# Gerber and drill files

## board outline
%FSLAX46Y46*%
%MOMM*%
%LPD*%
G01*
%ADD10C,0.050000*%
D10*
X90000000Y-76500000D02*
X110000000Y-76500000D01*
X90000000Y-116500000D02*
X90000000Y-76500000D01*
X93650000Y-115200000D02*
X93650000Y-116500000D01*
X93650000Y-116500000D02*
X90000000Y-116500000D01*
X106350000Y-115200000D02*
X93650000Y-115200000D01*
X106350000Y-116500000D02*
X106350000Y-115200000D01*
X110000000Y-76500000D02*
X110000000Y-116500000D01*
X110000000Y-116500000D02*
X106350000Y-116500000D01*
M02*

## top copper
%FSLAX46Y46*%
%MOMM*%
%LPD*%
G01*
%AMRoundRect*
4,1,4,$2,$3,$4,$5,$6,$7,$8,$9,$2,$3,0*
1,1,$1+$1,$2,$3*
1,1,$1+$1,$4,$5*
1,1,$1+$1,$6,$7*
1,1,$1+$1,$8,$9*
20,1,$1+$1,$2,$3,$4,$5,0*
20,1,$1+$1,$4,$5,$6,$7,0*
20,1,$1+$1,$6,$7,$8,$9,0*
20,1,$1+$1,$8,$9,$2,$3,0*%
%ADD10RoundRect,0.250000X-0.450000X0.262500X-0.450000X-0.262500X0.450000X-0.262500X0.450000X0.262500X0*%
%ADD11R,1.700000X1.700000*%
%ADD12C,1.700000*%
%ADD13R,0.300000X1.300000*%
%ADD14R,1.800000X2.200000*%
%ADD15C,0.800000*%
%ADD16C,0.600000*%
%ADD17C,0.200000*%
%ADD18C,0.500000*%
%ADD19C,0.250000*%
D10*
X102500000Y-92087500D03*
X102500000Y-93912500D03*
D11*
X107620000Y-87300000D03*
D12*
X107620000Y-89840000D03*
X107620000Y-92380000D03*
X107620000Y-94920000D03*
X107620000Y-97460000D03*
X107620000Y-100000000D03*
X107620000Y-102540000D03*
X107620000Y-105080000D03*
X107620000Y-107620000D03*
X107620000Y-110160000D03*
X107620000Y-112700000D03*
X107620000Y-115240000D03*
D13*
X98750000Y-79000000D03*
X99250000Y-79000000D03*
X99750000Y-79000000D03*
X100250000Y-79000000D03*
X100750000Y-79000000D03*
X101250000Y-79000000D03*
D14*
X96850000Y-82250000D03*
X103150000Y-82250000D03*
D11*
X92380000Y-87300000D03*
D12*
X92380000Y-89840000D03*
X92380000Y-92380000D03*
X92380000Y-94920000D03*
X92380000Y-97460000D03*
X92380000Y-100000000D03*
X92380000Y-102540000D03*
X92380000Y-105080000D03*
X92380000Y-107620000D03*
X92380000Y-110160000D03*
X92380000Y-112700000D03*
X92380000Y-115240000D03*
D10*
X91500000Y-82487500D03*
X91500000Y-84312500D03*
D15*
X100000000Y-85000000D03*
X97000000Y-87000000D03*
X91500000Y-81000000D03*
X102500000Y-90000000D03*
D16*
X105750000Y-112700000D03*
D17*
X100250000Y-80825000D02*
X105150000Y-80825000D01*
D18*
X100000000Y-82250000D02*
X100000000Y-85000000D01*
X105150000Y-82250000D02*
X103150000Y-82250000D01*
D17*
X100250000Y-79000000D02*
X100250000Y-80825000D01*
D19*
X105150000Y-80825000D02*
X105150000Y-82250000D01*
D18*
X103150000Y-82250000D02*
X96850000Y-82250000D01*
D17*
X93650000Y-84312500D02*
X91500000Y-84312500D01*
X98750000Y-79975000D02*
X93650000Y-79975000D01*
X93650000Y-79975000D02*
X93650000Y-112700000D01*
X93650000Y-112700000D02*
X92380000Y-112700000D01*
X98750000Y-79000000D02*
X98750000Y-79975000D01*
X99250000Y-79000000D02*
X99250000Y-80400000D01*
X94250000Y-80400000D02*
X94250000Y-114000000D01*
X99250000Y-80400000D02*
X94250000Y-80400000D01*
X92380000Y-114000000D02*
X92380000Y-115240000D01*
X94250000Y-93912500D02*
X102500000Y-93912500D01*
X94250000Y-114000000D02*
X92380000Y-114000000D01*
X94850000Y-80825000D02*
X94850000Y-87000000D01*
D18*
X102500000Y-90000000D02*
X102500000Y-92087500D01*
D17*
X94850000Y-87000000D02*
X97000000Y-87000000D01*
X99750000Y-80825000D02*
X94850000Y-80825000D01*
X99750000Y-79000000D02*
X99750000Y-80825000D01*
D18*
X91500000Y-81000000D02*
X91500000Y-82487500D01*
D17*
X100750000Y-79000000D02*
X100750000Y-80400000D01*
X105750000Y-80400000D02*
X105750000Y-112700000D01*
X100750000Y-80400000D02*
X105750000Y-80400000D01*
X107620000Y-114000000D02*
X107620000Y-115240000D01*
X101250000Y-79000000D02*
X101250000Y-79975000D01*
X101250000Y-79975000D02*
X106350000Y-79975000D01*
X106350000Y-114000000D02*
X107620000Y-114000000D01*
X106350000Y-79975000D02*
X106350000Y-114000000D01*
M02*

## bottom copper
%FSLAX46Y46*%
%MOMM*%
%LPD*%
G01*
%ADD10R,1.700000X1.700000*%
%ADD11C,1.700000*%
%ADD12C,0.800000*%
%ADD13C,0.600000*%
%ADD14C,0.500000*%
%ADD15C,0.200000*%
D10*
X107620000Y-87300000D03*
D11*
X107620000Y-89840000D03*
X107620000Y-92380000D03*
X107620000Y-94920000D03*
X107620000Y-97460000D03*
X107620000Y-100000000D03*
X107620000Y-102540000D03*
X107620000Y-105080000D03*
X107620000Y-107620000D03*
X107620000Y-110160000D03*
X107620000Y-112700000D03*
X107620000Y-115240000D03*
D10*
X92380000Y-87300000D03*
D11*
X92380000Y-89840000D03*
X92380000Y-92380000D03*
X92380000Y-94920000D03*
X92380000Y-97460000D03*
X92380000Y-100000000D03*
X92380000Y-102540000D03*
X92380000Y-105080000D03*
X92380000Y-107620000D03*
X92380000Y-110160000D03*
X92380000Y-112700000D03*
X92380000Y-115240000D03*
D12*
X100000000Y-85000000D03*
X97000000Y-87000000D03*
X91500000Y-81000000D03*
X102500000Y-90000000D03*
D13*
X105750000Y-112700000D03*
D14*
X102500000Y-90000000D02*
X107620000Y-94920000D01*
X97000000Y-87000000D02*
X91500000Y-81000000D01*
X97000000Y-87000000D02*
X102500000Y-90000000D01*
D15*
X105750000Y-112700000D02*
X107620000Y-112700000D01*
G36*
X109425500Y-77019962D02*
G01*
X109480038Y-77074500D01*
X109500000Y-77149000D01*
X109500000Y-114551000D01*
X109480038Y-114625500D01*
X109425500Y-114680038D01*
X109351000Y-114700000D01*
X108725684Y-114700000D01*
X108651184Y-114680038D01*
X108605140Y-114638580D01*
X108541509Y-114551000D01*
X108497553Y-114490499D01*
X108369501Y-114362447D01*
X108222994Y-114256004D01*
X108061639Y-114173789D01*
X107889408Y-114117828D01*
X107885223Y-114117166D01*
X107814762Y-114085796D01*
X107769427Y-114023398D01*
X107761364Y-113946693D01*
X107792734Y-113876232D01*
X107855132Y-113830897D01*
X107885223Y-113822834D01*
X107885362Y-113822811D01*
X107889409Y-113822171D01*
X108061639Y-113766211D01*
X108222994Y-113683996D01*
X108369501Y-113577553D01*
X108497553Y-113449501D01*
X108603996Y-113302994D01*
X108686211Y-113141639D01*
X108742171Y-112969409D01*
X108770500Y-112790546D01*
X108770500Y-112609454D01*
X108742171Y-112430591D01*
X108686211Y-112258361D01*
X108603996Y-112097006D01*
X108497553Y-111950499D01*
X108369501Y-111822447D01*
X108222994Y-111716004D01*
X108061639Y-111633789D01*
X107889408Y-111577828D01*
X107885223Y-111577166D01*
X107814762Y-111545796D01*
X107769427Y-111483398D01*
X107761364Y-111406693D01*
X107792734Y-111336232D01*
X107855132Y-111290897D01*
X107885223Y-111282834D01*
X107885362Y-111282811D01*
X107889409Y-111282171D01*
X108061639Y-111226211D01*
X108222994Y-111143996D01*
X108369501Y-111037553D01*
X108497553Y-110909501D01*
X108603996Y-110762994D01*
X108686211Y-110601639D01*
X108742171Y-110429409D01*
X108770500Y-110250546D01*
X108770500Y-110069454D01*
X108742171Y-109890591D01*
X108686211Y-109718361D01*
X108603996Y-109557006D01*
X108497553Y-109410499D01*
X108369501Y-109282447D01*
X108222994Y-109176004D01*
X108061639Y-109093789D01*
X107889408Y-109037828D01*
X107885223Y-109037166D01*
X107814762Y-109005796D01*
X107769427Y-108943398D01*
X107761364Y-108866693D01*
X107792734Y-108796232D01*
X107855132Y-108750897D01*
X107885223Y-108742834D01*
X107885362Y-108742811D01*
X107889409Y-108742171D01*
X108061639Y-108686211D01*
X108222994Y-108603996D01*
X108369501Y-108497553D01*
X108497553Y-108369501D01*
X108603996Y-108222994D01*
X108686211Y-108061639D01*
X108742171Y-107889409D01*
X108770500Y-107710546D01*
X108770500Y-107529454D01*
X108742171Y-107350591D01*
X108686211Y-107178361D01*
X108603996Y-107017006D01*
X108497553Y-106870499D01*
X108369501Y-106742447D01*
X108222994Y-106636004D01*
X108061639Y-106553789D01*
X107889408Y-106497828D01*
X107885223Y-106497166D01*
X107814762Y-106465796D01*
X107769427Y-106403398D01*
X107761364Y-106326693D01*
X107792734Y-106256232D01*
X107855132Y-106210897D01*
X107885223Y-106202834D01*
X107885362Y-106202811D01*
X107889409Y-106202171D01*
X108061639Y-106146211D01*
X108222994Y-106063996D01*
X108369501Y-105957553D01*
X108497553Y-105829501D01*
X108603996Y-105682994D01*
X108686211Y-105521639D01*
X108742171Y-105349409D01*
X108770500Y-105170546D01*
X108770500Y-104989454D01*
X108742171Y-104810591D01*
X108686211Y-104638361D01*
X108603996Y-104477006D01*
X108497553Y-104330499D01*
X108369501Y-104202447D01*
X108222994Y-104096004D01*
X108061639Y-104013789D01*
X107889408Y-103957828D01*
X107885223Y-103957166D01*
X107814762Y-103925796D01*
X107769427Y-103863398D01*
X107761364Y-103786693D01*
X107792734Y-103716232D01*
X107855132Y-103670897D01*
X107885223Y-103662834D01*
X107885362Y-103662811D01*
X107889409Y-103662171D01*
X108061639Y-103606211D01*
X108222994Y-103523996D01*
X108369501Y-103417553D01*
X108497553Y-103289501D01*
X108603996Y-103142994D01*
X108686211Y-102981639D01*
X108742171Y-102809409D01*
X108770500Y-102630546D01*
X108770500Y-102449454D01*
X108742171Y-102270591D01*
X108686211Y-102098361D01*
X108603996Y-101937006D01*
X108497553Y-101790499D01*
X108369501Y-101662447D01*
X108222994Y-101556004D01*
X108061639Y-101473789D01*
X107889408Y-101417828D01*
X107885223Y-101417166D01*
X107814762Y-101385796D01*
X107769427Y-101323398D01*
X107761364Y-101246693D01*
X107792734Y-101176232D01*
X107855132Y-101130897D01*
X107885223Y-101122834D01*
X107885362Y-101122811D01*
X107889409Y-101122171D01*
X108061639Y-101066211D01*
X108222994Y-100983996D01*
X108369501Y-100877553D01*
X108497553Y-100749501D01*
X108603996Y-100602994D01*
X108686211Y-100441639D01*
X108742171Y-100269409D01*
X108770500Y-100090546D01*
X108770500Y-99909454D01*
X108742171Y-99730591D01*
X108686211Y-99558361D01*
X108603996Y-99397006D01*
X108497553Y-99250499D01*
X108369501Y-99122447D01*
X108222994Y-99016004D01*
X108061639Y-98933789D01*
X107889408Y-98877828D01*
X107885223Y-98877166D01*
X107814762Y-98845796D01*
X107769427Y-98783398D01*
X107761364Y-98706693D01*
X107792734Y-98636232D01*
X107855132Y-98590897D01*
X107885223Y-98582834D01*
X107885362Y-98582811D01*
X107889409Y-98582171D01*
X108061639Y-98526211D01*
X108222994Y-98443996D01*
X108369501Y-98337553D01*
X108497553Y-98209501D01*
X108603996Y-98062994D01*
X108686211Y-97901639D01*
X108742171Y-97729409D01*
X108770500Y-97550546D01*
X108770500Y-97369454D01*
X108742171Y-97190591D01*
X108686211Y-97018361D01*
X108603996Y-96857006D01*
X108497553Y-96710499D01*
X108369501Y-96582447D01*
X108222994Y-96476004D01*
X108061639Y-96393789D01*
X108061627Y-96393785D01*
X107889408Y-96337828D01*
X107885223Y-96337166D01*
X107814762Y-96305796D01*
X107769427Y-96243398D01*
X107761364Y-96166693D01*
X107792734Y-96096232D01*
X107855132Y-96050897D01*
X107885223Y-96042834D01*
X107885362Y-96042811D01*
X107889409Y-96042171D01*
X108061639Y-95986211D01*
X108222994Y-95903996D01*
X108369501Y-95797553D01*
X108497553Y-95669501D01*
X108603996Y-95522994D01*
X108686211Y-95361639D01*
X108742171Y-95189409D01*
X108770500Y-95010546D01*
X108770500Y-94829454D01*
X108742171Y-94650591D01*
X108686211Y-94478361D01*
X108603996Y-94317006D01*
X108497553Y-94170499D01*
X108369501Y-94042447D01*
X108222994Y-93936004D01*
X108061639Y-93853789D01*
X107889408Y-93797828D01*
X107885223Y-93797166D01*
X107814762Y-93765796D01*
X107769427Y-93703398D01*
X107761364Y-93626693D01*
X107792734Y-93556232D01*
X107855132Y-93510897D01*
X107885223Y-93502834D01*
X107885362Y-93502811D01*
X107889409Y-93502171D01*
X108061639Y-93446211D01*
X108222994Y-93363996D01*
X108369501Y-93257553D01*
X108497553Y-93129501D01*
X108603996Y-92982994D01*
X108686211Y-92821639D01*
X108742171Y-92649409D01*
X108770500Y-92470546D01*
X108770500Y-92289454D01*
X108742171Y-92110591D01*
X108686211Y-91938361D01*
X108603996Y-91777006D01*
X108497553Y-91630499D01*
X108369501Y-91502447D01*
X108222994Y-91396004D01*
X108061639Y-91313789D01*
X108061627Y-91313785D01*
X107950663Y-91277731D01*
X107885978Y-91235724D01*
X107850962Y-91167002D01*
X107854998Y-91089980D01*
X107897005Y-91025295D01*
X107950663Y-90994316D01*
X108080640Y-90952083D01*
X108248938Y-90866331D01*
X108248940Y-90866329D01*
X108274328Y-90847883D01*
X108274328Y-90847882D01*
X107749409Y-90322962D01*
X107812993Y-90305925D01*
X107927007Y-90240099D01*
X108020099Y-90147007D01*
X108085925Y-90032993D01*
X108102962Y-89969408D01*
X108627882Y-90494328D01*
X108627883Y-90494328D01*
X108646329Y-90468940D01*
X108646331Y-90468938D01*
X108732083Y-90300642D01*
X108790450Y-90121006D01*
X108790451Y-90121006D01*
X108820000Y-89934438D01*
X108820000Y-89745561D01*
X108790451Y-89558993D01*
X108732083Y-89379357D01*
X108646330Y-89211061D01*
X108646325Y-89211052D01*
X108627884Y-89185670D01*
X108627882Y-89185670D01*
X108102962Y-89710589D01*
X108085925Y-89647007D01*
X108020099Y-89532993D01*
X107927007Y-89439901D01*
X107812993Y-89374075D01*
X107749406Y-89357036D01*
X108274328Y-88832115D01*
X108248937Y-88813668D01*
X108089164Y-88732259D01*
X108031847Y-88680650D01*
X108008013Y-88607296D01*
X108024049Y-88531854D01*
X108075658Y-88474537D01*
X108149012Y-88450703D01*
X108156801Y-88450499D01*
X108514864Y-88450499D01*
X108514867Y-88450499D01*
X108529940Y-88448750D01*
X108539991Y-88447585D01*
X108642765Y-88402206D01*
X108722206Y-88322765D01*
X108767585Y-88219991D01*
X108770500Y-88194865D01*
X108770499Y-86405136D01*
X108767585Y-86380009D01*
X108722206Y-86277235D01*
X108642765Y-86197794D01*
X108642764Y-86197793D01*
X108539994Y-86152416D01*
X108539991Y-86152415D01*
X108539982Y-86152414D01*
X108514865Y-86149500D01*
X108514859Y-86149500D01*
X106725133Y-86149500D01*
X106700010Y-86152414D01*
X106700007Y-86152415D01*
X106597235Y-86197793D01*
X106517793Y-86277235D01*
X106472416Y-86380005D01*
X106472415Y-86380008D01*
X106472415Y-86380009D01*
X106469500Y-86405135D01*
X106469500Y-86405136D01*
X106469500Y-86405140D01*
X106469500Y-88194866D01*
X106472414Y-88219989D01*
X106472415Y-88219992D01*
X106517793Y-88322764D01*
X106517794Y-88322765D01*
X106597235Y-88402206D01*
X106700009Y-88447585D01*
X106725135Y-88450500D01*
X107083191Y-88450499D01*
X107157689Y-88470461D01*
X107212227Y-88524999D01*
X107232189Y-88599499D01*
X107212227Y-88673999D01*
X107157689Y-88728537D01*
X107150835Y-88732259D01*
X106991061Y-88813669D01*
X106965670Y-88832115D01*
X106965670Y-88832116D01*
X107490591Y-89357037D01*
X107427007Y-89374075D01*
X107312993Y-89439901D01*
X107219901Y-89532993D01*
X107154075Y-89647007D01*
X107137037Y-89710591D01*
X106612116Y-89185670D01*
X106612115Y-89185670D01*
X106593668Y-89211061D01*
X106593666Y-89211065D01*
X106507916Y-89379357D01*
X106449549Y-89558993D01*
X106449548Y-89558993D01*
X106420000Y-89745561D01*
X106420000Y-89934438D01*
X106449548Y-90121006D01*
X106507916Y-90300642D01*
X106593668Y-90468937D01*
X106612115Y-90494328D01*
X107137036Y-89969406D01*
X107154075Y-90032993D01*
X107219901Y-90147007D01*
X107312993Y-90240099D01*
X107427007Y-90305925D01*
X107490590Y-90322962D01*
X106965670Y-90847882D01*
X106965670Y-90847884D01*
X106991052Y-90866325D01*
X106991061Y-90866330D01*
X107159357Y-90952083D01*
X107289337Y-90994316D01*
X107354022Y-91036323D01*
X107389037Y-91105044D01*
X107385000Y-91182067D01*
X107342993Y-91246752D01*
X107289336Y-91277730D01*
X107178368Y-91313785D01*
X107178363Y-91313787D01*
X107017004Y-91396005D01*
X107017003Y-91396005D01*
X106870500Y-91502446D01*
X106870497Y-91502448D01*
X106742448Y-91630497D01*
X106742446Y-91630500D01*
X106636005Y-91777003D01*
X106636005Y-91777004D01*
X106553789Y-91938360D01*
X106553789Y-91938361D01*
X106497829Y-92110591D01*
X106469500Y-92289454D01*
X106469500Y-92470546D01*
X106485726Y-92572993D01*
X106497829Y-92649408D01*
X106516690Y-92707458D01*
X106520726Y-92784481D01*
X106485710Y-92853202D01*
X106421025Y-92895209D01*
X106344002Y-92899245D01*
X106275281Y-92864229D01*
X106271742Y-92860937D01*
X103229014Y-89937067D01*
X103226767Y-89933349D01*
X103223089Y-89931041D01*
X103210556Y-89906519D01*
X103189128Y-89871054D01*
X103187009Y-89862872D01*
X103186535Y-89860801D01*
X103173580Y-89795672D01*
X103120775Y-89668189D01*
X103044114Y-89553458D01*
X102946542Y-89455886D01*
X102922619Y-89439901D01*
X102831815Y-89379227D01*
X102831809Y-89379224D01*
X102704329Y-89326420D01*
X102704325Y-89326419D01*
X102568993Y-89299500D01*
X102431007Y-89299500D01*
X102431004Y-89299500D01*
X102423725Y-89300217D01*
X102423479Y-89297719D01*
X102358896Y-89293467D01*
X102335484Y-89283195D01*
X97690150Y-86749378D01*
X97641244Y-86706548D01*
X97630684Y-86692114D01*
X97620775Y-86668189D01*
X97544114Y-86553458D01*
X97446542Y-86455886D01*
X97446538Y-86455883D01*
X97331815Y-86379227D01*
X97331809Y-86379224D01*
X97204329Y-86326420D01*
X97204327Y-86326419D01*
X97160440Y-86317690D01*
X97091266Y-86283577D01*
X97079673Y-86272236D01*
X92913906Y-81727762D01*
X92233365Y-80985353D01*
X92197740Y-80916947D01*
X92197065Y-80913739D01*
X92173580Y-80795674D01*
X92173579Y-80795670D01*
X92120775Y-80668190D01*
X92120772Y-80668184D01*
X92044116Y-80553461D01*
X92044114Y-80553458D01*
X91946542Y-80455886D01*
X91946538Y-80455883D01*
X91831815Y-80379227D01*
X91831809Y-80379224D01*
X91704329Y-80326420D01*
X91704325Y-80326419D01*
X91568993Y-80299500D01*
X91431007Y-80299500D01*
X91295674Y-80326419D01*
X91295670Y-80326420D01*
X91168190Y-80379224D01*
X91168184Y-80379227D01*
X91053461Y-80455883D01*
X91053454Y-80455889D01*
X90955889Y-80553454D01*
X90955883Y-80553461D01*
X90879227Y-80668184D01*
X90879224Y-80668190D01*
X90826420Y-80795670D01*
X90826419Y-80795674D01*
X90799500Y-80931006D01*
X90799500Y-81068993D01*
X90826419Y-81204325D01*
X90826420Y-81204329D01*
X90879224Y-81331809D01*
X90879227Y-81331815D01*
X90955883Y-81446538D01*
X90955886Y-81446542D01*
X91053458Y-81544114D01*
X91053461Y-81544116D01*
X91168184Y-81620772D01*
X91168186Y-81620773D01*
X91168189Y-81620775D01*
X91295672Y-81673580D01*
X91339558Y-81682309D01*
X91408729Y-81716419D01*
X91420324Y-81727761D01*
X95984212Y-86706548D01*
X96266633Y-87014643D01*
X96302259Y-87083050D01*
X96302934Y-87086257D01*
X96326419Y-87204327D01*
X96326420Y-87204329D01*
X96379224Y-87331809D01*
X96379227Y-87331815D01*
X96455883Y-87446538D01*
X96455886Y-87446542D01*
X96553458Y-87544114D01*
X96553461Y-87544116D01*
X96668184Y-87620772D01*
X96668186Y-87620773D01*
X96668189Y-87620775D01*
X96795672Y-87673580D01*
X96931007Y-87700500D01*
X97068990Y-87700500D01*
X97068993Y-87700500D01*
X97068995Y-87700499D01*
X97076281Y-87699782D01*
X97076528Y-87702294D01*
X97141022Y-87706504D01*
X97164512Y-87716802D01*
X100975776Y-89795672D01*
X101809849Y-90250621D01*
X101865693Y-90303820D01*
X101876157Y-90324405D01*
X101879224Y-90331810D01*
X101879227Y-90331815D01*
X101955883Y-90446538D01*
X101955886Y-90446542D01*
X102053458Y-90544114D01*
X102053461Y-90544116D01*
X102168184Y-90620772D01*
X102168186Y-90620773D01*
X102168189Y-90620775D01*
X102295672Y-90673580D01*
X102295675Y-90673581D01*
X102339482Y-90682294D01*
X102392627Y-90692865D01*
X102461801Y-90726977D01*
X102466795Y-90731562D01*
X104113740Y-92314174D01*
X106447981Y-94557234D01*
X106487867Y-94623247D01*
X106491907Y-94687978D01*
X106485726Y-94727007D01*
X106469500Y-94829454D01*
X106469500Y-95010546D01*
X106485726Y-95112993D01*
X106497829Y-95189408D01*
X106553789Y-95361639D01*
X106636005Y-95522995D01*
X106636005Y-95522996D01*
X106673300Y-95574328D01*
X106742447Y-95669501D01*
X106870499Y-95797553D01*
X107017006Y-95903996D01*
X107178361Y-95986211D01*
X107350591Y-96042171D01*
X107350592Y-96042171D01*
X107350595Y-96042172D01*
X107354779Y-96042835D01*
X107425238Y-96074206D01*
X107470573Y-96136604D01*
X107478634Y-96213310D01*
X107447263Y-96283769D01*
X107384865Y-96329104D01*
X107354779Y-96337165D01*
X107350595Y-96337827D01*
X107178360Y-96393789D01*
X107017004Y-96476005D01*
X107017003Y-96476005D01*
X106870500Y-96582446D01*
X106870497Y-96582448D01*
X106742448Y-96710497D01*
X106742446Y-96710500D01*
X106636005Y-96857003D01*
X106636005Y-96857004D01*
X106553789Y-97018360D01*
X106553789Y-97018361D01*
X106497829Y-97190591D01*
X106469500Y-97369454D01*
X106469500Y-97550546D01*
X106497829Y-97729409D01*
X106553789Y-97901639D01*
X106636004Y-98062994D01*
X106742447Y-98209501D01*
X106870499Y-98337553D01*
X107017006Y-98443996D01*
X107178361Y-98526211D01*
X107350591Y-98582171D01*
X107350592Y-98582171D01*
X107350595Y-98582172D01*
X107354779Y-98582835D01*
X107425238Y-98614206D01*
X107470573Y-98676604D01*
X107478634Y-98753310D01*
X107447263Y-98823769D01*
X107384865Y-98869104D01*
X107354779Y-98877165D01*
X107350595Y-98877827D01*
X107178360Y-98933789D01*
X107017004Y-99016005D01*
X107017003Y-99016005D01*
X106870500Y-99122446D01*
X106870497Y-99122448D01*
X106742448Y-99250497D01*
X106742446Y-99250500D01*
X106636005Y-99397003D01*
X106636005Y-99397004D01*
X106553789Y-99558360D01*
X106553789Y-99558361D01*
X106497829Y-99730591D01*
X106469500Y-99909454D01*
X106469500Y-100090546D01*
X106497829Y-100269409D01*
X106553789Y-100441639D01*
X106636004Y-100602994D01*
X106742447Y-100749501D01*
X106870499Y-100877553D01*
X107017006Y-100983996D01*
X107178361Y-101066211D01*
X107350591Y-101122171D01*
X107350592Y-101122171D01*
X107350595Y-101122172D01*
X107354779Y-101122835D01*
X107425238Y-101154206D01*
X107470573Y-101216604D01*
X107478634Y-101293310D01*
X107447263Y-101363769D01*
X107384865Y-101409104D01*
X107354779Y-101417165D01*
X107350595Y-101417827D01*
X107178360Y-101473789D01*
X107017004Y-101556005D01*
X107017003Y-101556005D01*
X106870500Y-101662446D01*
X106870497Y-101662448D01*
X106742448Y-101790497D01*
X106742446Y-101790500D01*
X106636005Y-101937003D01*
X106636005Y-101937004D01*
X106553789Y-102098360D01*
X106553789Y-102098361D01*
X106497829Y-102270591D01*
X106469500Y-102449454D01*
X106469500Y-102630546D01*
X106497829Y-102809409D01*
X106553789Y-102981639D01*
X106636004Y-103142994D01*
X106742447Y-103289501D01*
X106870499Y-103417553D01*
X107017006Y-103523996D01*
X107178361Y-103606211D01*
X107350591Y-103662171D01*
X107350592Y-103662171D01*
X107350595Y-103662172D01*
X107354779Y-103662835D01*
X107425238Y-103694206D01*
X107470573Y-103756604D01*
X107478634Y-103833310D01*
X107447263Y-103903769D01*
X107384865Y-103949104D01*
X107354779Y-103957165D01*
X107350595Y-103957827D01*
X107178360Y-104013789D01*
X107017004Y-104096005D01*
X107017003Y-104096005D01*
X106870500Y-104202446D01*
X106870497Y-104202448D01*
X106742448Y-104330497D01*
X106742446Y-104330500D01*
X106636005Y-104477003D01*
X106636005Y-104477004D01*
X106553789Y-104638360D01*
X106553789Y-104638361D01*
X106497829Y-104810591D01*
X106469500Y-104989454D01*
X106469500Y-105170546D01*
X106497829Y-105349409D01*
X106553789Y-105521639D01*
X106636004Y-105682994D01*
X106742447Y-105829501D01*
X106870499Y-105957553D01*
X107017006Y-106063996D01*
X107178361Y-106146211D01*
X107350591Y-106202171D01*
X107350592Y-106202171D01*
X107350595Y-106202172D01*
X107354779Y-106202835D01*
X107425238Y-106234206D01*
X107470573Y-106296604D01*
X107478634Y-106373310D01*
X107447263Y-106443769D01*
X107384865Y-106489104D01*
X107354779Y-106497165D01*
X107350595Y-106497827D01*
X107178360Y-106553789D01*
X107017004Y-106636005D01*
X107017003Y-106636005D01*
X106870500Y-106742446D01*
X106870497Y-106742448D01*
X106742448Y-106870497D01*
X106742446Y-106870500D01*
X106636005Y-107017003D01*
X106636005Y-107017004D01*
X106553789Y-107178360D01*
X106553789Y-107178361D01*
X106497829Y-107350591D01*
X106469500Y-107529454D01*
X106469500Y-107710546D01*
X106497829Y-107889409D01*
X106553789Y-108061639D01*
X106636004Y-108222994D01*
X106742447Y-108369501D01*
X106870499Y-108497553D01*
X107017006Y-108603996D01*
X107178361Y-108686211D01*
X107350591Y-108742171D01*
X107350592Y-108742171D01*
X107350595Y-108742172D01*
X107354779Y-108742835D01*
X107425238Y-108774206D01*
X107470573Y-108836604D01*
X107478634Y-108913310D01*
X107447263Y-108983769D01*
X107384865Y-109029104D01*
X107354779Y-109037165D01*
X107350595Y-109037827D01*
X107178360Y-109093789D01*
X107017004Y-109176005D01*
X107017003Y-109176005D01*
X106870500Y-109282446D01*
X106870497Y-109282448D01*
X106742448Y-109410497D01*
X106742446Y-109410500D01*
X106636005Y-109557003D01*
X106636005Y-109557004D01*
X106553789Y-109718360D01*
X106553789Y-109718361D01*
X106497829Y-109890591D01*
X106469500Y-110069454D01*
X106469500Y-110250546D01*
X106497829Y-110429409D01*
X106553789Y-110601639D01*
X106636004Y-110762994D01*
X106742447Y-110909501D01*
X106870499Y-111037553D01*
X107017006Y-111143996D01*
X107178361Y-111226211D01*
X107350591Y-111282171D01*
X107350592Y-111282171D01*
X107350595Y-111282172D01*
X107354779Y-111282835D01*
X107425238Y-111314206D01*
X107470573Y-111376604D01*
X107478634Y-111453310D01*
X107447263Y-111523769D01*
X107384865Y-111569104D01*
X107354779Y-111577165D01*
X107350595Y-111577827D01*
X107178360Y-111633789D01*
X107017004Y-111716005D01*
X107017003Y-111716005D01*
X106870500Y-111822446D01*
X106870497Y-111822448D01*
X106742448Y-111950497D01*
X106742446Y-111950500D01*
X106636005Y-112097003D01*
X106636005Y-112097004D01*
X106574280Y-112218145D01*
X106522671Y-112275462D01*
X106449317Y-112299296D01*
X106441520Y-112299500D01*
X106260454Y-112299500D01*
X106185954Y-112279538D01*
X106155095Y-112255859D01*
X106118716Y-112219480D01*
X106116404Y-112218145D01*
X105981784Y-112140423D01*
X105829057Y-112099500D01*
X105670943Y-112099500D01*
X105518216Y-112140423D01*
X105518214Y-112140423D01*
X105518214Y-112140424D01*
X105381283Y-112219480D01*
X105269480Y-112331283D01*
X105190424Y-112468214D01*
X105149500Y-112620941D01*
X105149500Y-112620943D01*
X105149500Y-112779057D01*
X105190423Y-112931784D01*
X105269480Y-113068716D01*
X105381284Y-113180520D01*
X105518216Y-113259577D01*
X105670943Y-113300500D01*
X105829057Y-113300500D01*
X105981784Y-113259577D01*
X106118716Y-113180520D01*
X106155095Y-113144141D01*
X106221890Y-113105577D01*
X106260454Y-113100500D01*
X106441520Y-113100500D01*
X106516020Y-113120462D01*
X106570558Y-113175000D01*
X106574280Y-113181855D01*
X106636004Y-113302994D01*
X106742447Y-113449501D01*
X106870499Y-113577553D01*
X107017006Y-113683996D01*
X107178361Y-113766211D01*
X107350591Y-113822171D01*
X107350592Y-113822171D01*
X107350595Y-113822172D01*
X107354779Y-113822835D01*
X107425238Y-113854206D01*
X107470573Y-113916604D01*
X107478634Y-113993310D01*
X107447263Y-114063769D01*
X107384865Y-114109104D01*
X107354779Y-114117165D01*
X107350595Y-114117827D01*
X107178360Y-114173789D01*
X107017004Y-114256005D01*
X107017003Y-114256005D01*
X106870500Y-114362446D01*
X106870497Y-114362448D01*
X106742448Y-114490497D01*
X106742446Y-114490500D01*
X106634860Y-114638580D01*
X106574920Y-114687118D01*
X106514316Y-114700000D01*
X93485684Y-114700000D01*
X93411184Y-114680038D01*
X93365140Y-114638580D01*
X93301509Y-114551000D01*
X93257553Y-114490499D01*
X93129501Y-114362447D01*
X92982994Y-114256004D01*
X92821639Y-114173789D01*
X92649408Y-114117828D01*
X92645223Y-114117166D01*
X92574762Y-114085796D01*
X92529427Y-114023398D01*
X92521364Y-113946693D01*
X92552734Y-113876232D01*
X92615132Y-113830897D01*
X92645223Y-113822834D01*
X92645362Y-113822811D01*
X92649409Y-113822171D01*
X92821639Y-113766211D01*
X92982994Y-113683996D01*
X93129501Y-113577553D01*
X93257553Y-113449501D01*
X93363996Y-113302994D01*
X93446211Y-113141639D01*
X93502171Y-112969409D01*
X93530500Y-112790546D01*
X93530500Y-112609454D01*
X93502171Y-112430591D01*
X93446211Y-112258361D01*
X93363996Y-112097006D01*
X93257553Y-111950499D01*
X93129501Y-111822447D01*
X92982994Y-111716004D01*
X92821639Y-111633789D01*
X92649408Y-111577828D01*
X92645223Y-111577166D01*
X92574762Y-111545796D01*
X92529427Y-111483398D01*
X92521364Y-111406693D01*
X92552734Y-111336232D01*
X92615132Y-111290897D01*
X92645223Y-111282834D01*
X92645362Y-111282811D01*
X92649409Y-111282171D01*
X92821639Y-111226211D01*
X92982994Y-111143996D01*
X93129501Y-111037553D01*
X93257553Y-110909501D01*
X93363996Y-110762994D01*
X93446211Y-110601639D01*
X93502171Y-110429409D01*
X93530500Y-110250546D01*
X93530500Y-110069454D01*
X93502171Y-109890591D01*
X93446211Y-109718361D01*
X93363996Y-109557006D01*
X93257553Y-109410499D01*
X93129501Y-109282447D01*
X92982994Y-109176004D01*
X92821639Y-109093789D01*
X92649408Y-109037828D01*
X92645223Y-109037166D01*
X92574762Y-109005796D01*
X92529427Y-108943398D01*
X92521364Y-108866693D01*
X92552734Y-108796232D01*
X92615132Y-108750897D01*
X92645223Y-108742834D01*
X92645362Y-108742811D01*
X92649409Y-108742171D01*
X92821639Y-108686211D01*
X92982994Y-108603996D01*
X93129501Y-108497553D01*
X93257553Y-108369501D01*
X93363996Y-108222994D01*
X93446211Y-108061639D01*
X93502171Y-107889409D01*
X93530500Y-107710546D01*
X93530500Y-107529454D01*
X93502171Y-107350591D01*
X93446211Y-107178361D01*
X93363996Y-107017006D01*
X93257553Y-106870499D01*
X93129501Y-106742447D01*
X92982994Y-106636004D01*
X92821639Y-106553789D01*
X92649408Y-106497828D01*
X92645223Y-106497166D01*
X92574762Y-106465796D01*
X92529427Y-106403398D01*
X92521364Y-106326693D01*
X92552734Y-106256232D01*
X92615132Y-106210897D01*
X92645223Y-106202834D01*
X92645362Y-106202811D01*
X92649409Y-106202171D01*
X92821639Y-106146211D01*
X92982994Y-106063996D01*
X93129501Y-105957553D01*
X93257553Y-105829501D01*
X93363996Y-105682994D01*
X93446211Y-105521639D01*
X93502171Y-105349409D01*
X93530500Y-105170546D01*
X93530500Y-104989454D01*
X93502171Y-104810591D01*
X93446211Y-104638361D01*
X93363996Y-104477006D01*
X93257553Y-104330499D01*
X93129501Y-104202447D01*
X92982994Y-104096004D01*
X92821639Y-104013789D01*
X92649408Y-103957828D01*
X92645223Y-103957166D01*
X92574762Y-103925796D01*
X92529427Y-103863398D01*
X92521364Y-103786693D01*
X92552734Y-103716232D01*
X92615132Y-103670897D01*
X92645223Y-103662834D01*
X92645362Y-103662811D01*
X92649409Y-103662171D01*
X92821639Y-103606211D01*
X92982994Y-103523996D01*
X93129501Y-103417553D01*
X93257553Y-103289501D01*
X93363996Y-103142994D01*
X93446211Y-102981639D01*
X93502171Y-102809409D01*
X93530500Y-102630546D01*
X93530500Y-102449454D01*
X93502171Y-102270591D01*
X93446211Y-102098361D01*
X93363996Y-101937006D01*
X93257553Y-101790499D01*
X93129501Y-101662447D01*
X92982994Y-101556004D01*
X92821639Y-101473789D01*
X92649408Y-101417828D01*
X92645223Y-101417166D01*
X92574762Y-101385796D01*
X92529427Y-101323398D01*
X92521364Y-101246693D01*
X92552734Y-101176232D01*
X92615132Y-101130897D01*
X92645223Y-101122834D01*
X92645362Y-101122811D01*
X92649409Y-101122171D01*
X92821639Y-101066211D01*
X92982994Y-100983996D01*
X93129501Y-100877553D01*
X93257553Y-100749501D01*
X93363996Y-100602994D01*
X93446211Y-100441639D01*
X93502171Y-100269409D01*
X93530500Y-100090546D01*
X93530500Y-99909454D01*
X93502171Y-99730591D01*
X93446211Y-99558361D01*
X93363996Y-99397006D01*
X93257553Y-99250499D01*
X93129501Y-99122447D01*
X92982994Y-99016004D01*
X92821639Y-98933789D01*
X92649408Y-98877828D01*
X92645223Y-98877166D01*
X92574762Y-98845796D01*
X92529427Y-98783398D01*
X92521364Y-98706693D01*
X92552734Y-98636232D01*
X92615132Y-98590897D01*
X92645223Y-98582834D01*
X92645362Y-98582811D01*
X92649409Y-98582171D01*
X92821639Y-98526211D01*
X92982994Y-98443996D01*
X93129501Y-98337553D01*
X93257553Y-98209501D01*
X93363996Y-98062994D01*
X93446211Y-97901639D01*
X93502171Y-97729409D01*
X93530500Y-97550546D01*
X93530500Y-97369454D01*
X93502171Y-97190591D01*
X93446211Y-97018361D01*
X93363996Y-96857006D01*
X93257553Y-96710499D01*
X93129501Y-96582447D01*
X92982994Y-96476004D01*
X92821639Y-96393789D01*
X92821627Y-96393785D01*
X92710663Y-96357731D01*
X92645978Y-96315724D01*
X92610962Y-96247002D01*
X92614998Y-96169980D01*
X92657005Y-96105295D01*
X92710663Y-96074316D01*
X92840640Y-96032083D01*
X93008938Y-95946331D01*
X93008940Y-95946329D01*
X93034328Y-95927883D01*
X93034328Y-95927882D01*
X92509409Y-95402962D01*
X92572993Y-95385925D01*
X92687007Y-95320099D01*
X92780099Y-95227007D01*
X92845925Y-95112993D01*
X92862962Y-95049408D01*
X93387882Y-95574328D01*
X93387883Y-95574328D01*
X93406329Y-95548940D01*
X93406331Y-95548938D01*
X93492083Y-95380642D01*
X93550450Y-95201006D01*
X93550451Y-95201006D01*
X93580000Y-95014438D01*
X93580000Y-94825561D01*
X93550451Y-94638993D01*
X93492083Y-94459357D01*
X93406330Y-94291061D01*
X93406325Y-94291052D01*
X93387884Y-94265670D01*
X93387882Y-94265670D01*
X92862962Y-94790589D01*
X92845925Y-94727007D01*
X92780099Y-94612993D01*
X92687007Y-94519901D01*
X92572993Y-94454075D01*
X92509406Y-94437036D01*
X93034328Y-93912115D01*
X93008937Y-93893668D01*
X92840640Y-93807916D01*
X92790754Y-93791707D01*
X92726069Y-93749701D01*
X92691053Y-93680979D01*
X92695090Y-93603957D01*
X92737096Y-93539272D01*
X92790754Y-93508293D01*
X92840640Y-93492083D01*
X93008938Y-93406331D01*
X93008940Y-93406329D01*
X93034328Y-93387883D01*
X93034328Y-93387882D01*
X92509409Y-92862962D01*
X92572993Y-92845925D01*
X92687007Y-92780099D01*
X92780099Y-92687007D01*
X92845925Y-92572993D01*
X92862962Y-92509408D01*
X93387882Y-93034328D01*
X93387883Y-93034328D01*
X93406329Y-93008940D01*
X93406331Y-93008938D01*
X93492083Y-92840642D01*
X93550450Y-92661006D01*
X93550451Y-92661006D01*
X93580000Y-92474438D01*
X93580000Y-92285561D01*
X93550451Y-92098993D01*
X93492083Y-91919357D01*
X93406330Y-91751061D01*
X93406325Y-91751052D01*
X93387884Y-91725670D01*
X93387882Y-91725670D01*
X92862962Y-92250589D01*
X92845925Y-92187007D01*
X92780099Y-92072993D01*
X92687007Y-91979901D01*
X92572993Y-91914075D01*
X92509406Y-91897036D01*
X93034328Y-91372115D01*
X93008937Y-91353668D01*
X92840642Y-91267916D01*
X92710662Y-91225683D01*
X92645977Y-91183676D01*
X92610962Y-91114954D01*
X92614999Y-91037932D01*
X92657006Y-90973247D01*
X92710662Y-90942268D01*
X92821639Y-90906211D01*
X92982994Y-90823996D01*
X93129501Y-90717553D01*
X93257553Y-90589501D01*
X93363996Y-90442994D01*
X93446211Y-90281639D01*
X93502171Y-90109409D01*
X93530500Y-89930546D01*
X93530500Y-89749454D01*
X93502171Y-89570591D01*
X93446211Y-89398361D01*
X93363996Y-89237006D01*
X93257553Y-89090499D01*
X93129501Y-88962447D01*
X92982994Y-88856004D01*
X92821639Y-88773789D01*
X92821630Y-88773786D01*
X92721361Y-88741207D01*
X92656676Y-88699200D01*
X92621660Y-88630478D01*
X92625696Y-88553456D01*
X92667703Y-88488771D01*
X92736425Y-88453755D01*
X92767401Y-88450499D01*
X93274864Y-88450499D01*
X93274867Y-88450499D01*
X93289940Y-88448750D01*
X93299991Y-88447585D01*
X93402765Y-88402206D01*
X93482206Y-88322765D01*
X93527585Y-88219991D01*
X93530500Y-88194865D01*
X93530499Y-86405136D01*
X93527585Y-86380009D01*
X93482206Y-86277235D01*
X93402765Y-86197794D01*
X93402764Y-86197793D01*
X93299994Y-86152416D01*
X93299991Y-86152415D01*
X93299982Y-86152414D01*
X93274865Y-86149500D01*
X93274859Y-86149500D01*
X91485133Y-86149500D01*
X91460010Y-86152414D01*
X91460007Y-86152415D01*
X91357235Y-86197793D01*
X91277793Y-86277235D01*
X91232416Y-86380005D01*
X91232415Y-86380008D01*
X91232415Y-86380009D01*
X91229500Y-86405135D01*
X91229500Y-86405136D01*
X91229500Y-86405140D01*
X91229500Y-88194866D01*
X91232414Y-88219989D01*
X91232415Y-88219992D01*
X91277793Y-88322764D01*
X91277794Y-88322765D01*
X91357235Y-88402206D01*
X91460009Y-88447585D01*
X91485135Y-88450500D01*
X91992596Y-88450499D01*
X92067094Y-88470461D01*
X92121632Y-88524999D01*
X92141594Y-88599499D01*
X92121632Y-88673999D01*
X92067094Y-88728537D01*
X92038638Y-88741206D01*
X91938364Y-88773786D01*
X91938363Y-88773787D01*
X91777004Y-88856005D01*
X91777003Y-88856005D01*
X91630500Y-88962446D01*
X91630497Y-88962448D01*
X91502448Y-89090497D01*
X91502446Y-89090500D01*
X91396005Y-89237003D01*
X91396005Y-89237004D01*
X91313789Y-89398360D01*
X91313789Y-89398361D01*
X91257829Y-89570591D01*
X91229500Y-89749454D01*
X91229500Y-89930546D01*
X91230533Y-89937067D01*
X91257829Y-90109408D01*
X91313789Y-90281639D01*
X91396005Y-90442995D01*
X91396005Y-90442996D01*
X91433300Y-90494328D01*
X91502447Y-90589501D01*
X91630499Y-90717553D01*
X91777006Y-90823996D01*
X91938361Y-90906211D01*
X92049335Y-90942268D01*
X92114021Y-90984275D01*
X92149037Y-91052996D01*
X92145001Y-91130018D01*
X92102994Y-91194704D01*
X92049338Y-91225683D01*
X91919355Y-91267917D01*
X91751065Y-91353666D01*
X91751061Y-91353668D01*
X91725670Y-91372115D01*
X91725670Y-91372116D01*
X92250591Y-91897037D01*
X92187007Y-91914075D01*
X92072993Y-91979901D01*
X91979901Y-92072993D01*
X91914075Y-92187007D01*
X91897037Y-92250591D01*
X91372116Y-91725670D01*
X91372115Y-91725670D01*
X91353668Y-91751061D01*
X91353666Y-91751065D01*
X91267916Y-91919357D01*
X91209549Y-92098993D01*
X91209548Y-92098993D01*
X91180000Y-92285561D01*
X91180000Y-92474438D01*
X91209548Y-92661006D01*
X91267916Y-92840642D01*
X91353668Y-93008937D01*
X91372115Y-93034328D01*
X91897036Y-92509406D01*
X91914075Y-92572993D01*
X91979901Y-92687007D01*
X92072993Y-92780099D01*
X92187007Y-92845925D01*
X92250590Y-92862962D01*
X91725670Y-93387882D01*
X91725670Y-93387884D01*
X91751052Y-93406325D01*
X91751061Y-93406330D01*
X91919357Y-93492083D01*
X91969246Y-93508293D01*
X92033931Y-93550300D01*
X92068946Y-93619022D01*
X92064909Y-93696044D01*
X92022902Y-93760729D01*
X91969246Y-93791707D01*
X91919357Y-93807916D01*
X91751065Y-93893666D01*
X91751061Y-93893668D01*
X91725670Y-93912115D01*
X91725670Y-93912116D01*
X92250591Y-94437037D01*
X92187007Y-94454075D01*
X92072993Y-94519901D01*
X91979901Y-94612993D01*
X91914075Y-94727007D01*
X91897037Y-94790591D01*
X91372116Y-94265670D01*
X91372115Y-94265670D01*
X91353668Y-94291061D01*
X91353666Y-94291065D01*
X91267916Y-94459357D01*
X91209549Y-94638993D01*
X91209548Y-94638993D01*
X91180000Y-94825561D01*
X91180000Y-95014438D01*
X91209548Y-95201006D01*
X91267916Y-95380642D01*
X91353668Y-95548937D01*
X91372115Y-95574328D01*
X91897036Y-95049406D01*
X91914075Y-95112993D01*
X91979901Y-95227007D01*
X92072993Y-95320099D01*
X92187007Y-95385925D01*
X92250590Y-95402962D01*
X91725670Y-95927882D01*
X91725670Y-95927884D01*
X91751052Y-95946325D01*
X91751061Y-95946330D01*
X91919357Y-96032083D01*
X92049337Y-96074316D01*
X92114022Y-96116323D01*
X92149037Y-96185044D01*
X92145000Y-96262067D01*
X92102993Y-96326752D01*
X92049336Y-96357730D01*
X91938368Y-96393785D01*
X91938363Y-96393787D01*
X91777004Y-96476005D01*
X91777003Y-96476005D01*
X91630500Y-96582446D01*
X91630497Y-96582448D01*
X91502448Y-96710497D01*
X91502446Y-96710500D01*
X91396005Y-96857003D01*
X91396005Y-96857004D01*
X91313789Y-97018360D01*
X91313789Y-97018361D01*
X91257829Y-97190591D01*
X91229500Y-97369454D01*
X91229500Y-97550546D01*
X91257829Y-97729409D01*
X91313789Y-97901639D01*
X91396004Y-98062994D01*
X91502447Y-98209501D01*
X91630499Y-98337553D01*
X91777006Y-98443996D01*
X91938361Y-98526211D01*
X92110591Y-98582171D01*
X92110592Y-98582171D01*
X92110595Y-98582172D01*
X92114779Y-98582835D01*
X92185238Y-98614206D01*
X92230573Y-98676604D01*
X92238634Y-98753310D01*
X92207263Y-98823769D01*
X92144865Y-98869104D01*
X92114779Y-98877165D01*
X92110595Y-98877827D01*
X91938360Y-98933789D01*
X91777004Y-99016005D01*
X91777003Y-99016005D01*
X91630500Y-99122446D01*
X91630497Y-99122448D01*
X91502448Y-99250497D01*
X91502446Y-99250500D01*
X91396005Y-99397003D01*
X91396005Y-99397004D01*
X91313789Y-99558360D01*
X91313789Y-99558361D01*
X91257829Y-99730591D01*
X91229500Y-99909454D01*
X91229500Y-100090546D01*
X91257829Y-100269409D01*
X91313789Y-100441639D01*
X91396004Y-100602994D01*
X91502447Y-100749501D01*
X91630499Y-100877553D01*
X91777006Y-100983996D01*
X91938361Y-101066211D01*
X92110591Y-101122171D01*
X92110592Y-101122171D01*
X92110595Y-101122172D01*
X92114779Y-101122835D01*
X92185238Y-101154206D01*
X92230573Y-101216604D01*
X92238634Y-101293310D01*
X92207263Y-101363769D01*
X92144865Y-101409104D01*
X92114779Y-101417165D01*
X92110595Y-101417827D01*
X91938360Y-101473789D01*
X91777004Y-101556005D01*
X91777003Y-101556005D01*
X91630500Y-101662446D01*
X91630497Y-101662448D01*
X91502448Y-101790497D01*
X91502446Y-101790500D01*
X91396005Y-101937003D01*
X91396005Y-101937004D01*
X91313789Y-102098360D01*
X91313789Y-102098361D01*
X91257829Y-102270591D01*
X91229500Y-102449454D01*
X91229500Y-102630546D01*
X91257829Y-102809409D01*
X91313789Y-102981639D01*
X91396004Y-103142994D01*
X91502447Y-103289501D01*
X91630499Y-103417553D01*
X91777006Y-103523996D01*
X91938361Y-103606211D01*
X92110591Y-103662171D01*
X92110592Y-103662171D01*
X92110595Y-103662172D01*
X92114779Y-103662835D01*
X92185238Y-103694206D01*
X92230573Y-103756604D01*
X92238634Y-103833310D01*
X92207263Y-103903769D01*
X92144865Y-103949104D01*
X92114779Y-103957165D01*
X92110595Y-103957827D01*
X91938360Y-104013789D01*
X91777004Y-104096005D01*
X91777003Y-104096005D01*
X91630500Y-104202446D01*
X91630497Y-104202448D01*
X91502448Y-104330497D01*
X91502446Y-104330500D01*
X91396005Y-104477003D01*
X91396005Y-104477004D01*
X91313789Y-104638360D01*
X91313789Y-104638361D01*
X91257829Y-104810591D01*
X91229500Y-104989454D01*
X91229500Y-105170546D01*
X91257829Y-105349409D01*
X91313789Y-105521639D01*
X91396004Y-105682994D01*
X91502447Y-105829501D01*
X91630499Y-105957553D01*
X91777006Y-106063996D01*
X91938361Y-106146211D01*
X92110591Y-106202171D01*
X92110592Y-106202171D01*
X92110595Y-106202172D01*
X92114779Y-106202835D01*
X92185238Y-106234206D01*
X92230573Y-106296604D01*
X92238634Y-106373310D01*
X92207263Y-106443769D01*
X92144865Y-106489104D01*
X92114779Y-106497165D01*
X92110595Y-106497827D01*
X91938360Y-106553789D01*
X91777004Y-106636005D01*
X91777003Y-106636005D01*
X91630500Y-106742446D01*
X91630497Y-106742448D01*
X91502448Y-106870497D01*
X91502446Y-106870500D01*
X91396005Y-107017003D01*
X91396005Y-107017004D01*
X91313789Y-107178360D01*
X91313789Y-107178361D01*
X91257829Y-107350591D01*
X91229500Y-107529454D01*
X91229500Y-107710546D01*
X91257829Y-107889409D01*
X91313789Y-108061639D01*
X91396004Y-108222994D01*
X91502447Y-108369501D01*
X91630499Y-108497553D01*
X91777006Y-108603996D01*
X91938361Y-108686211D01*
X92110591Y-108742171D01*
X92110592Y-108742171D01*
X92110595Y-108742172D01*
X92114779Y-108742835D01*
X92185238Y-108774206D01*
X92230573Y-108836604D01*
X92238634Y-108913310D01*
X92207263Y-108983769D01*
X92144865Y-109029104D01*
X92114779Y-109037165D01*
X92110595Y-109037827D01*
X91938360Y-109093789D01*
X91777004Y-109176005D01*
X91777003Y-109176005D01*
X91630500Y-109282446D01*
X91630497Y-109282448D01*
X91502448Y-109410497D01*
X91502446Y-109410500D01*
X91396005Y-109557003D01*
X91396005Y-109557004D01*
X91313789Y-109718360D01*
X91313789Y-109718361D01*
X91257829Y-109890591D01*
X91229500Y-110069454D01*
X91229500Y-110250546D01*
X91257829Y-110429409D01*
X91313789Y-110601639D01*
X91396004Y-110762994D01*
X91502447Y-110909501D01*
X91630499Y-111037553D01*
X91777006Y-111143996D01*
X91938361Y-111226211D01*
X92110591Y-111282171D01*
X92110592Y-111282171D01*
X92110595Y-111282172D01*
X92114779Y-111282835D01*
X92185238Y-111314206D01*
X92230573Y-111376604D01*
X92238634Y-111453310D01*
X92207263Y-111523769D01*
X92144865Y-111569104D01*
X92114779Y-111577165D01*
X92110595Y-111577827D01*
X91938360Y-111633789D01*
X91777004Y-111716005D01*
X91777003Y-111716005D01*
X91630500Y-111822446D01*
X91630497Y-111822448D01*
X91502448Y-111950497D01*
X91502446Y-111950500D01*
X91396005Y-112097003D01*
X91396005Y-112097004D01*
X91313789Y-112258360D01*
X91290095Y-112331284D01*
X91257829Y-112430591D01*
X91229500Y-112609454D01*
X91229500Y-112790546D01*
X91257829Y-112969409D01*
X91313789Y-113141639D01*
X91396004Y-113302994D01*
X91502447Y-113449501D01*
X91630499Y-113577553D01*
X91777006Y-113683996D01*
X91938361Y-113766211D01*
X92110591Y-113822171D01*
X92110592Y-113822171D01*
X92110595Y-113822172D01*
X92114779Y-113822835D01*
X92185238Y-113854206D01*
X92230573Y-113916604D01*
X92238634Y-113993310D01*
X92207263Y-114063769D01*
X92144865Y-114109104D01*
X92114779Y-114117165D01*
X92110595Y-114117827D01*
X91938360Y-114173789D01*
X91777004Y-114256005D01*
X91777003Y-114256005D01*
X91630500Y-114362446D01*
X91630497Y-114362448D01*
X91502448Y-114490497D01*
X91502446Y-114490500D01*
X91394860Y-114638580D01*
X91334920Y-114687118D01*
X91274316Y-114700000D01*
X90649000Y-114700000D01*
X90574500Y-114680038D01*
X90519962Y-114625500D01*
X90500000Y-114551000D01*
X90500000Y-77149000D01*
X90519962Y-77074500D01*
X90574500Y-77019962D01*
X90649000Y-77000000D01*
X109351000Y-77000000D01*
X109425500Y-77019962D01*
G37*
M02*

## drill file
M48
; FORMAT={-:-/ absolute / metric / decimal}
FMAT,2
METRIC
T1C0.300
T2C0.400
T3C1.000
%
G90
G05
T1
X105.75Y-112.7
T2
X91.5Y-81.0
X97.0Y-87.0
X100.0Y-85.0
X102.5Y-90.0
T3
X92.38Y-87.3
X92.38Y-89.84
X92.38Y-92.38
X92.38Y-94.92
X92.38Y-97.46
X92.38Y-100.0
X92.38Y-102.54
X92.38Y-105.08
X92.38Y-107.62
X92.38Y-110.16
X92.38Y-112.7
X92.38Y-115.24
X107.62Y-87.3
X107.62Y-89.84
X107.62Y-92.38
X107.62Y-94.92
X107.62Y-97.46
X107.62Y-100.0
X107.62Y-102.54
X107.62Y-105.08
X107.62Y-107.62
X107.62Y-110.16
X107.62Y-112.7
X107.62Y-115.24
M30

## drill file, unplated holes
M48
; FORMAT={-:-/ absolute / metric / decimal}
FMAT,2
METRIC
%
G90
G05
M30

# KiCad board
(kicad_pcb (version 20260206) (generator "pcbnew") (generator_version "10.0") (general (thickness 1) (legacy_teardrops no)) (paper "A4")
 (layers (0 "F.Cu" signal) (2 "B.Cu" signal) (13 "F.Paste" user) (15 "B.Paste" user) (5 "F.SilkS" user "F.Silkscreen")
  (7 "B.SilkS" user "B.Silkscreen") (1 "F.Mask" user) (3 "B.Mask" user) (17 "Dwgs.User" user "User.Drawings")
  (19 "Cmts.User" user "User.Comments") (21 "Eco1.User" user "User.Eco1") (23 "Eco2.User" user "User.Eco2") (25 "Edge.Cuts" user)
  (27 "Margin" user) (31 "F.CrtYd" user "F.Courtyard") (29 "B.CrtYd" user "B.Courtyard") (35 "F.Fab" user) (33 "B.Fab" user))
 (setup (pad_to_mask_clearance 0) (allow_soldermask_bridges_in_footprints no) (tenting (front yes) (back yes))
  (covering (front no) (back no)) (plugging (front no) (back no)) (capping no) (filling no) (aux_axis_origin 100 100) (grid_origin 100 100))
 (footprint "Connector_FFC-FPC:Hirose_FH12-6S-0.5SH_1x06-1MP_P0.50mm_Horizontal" (layer "F.Cu") (at 100 80.85)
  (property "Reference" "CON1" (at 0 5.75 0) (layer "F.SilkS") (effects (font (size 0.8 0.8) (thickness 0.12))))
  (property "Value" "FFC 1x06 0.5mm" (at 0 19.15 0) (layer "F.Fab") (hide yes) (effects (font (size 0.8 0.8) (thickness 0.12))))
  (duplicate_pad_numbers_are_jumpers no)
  (pad "1" smd rect (at -1.25 -1.85) (size 0.3 1.3) (layers "F.Cu" "F.Mask" "F.Paste") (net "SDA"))
  (pad "2" smd rect (at -0.75 -1.85) (size 0.3 1.3) (layers "F.Cu" "F.Mask" "F.Paste") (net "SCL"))
  (pad "3" smd rect (at -0.25 -1.85) (size 0.3 1.3) (layers "F.Cu" "F.Mask" "F.Paste") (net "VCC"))
  (pad "4" smd rect (at 0.25 -1.85) (size 0.3 1.3) (layers "F.Cu" "F.Mask" "F.Paste") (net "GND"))
  (pad "5" smd rect (at 0.75 -1.85) (size 0.3 1.3) (layers "F.Cu" "F.Mask" "F.Paste") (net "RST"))
  (pad "6" smd rect (at 1.25 -1.85) (size 0.3 1.3) (layers "F.Cu" "F.Mask" "F.Paste") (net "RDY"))
  (pad "MP" smd rect (at -3.15 1.4) (size 1.8 2.2) (layers "F.Cu" "F.Mask" "F.Paste") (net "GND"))
  (pad "MP" smd rect (at 3.15 1.4) (size 1.8 2.2) (layers "F.Cu" "F.Mask" "F.Paste") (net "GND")))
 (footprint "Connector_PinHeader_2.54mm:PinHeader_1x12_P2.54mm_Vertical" (layer "F.Cu") (at 92.38 87.3)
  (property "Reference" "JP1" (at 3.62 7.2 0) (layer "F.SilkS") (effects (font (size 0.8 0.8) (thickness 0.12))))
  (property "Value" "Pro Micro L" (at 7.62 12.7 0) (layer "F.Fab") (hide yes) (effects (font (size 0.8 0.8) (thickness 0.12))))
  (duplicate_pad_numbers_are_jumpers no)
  (pad "1" thru_hole rect (at 0 0) (size 1.7 1.7) (drill 1) (layers "*.Cu" "*.Mask") (remove_unused_layers no)
   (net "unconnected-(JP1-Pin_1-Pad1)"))
  (pad "2" thru_hole circle (at 0 2.54) (size 1.7 1.7) (drill 1) (layers "*.Cu" "*.Mask") (remove_unused_layers no)
   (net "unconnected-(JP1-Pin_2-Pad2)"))
  (pad "3" thru_hole circle (at 0 5.08) (size 1.7 1.7) (drill 1) (layers "*.Cu" "*.Mask") (remove_unused_layers no) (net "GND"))
  (pad "4" thru_hole circle (at 0 7.62) (size 1.7 1.7) (drill 1) (layers "*.Cu" "*.Mask") (remove_unused_layers no) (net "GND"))
  (pad "5" thru_hole circle (at 0 10.16) (size 1.7 1.7) (drill 1) (layers "*.Cu" "*.Mask") (remove_unused_layers no)
   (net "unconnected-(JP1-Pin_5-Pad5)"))
  (pad "6" thru_hole circle (at 0 12.7) (size 1.7 1.7) (drill 1) (layers "*.Cu" "*.Mask") (remove_unused_layers no)
   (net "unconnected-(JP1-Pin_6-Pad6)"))
  (pad "7" thru_hole circle (at 0 15.24) (size 1.7 1.7) (drill 1) (layers "*.Cu" "*.Mask") (remove_unused_layers no)
   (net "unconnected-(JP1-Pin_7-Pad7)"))
  (pad "8" thru_hole circle (at 0 17.78) (size 1.7 1.7) (drill 1) (layers "*.Cu" "*.Mask") (remove_unused_layers no)
   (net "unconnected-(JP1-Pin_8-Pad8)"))
  (pad "9" thru_hole circle (at 0 20.32) (size 1.7 1.7) (drill 1) (layers "*.Cu" "*.Mask") (remove_unused_layers no)
   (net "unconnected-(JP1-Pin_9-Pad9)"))
  (pad "10" thru_hole circle (at 0 22.86) (size 1.7 1.7) (drill 1) (layers "*.Cu" "*.Mask") (remove_unused_layers no)
   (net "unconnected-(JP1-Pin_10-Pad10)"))
  (pad "11" thru_hole circle (at 0 25.4) (size 1.7 1.7) (drill 1) (layers "*.Cu" "*.Mask") (remove_unused_layers no) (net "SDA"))
  (pad "12" thru_hole circle (at 0 27.94) (size 1.7 1.7) (drill 1) (layers "*.Cu" "*.Mask") (remove_unused_layers no) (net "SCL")))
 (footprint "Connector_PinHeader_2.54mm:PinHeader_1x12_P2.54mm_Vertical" (layer "F.Cu") (at 107.62 87.3)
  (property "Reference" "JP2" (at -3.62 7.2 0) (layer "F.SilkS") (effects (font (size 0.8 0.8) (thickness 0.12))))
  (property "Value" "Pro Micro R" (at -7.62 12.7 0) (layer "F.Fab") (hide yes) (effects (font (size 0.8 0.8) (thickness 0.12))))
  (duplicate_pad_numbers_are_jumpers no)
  (pad "1" thru_hole rect (at 0 0) (size 1.7 1.7) (drill 1) (layers "*.Cu" "*.Mask") (remove_unused_layers no)
   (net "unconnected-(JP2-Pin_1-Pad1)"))
  (pad "2" thru_hole circle (at 0 2.54) (size 1.7 1.7) (drill 1) (layers "*.Cu" "*.Mask") (remove_unused_layers no) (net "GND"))
  (pad "3" thru_hole circle (at 0 5.08) (size 1.7 1.7) (drill 1) (layers "*.Cu" "*.Mask") (remove_unused_layers no)
   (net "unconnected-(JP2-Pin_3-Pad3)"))
  (pad "4" thru_hole circle (at 0 7.62) (size 1.7 1.7) (drill 1) (layers "*.Cu" "*.Mask") (remove_unused_layers no) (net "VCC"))
  (pad "5" thru_hole circle (at 0 10.16) (size 1.7 1.7) (drill 1) (layers "*.Cu" "*.Mask") (remove_unused_layers no)
   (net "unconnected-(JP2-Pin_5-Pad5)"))
  (pad "6" thru_hole circle (at 0 12.7) (size 1.7 1.7) (drill 1) (layers "*.Cu" "*.Mask") (remove_unused_layers no)
   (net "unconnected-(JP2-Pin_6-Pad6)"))
  (pad "7" thru_hole circle (at 0 15.24) (size 1.7 1.7) (drill 1) (layers "*.Cu" "*.Mask") (remove_unused_layers no)
   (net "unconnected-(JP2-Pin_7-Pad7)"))
  (pad "8" thru_hole circle (at 0 17.78) (size 1.7 1.7) (drill 1) (layers "*.Cu" "*.Mask") (remove_unused_layers no)
   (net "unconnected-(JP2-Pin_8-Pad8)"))
  (pad "9" thru_hole circle (at 0 20.32) (size 1.7 1.7) (drill 1) (layers "*.Cu" "*.Mask") (remove_unused_layers no)
   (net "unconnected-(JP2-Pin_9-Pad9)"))
  (pad "10" thru_hole circle (at 0 22.86) (size 1.7 1.7) (drill 1) (layers "*.Cu" "*.Mask") (remove_unused_layers no)
   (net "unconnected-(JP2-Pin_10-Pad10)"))
  (pad "11" thru_hole circle (at 0 25.4) (size 1.7 1.7) (drill 1) (layers "*.Cu" "*.Mask") (remove_unused_layers no) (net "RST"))
  (pad "12" thru_hole circle (at 0 27.94) (size 1.7 1.7) (drill 1) (layers "*.Cu" "*.Mask") (remove_unused_layers no) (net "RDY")))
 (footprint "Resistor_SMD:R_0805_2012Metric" (layer "F.Cu") (at 102.5 93 -90)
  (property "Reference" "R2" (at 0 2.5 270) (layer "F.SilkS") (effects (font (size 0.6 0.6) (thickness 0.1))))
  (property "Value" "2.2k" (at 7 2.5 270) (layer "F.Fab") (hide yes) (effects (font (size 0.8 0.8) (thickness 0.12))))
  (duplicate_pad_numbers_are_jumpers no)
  (pad "1" smd roundrect (at -0.9125 0 270) (size 1.025 1.4) (layers "F.Cu" "F.Mask" "F.Paste") (roundrect_rratio 0.243902) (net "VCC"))
  (pad "2" smd roundrect (at 0.9125 0 270) (size 1.025 1.4) (layers "F.Cu" "F.Mask" "F.Paste") (roundrect_rratio 0.243902) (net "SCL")))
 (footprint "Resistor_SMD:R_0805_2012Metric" (layer "F.Cu") (at 91.5 83.4 -90)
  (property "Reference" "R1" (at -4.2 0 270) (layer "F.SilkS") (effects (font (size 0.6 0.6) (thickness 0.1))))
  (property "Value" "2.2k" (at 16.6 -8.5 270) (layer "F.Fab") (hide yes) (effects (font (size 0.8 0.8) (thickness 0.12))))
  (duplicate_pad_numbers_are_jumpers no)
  (pad "1" smd roundrect (at -0.9125 0 270) (size 1.025 1.4) (layers "F.Cu" "F.Mask" "F.Paste") (roundrect_rratio 0.243902) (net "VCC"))
  (pad "2" smd roundrect (at 0.9125 0 270) (size 1.025 1.4) (layers "F.Cu" "F.Mask" "F.Paste") (roundrect_rratio 0.243902) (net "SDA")))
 (gr_line (start 90 76.5) (end 110 76.5) (stroke (width 0.05) (type default)) (layer "Edge.Cuts"))
 (gr_line (start 90 116.5) (end 90 76.5) (stroke (width 0.05) (type default)) (layer "Edge.Cuts"))
 (gr_line (start 93.65 115.2) (end 93.65 116.5) (stroke (width 0.05) (type default)) (layer "Edge.Cuts"))
 (gr_line (start 93.65 116.5) (end 90 116.5) (stroke (width 0.05) (type default)) (layer "Edge.Cuts"))
 (gr_line (start 106.35 115.2) (end 93.65 115.2) (stroke (width 0.05) (type default)) (layer "Edge.Cuts"))
 (gr_line (start 106.35 116.5) (end 106.35 115.2) (stroke (width 0.05) (type default)) (layer "Edge.Cuts"))
 (gr_line (start 110 76.5) (end 110 116.5) (stroke (width 0.05) (type default)) (layer "Edge.Cuts"))
 (gr_line (start 110 116.5) (end 106.35 116.5) (stroke (width 0.05) (type default)) (layer "Edge.Cuts"))
 (segment (start 105.15 82.25) (end 103.15 82.25) (width 0.5) (layer "F.Cu") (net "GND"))
 (segment (start 103.15 82.25) (end 96.85 82.25) (width 0.5) (layer "F.Cu") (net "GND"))
 (segment (start 100 82.25) (end 100 85) (width 0.5) (layer "F.Cu") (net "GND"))
 (segment (start 100.25 80.825) (end 105.15 80.825) (width 0.2) (layer "F.Cu") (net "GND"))
 (segment (start 100.25 79) (end 100.25 80.825) (width 0.2) (layer "F.Cu") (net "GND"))
 (segment (start 105.15 80.825) (end 105.15 82.25) (width 0.25) (layer "F.Cu") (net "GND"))
 (via (at 100 85) (size 0.8) (drill 0.4) (layers "F.Cu" "B.Cu") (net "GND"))
 (segment (start 93.65 84.3125) (end 91.5 84.3125) (width 0.2) (layer "F.Cu") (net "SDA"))
 (segment (start 98.75 79) (end 98.75 79.975) (width 0.2) (layer "F.Cu") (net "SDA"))
 (segment (start 93.65 112.7) (end 92.38 112.7) (width 0.2) (layer "F.Cu") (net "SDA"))
 (segment (start 98.75 79.975) (end 93.65 79.975) (width 0.2) (layer "F.Cu") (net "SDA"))
 (segment (start 93.65 79.975) (end 93.65 112.7) (width 0.2) (layer "F.Cu") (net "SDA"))
 (segment (start 99.25 80.4) (end 94.25 80.4) (width 0.2) (layer "F.Cu") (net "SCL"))
 (segment (start 94.25 93.9125) (end 102.5 93.9125) (width 0.2) (layer "F.Cu") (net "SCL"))
 (segment (start 92.38 114) (end 92.38 115.24) (width 0.2) (layer "F.Cu") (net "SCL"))
 (segment (start 94.25 114) (end 92.38 114) (width 0.2) (layer "F.Cu") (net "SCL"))
 (segment (start 94.25 80.4) (end 94.25 114) (width 0.2) (layer "F.Cu") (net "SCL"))
 (segment (start 99.25 79) (end 99.25 80.4) (width 0.2) (layer "F.Cu") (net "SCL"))
 (segment (start 102.5 90) (end 102.5 92.0875) (width 0.5) (layer "F.Cu") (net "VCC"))
 (segment (start 94.85 87) (end 97 87) (width 0.2) (layer "F.Cu") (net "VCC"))
 (segment (start 94.85 80.825) (end 94.85 87) (width 0.2) (layer "F.Cu") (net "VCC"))
 (segment (start 99.75 80.825) (end 94.85 80.825) (width 0.2) (layer "F.Cu") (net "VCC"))
 (segment (start 99.75 79) (end 99.75 80.825) (width 0.2) (layer "F.Cu") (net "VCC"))
 (segment (start 91.5 81) (end 91.5 82.4875) (width 0.5) (layer "F.Cu") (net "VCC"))
 (via (at 102.5 90) (size 0.8) (drill 0.4) (layers "F.Cu" "B.Cu") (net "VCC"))
 (via (at 97 87) (size 0.8) (drill 0.4) (layers "F.Cu" "B.Cu") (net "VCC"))
 (via (at 91.5 81) (size 0.8) (drill 0.4) (layers "F.Cu" "B.Cu") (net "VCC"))
 (segment (start 102.5 90) (end 107.62 94.92) (width 0.5) (layer "B.Cu") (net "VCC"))
 (segment (start 97 87) (end 102.5 90) (width 0.5) (layer "B.Cu") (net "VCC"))
 (segment (start 97 87) (end 91.5 81) (width 0.5) (layer "B.Cu") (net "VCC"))
 (segment (start 100.75 79) (end 100.75 80.4) (width 0.2) (layer "F.Cu") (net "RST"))
 (segment (start 105.75 80.4) (end 105.75 112.7) (width 0.2) (layer "F.Cu") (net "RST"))
 (segment (start 100.75 80.4) (end 105.75 80.4) (width 0.2) (layer "F.Cu") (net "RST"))
 (via (at 105.75 112.7) (size 0.6) (drill 0.3) (layers "F.Cu" "B.Cu") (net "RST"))
 (segment (start 105.75 112.7) (end 107.62 112.7) (width 0.2) (layer "B.Cu") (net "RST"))
 (segment (start 106.35 79.975) (end 106.35 114) (width 0.2) (layer "F.Cu") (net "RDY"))
 (segment (start 106.35 114) (end 107.62 114) (width 0.2) (layer "F.Cu") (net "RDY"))
 (segment (start 107.62 114) (end 107.62 115.24) (width 0.2) (layer "F.Cu") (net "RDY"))
 (segment (start 101.25 79) (end 101.25 79.975) (width 0.2) (layer "F.Cu") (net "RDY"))
 (segment (start 101.25 79.975) (end 106.35 79.975) (width 0.2) (layer "F.Cu") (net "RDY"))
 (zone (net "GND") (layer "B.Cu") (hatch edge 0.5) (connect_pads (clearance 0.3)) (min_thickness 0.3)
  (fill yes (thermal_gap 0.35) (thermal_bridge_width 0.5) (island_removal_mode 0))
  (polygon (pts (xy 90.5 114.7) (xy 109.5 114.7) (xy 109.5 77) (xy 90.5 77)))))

